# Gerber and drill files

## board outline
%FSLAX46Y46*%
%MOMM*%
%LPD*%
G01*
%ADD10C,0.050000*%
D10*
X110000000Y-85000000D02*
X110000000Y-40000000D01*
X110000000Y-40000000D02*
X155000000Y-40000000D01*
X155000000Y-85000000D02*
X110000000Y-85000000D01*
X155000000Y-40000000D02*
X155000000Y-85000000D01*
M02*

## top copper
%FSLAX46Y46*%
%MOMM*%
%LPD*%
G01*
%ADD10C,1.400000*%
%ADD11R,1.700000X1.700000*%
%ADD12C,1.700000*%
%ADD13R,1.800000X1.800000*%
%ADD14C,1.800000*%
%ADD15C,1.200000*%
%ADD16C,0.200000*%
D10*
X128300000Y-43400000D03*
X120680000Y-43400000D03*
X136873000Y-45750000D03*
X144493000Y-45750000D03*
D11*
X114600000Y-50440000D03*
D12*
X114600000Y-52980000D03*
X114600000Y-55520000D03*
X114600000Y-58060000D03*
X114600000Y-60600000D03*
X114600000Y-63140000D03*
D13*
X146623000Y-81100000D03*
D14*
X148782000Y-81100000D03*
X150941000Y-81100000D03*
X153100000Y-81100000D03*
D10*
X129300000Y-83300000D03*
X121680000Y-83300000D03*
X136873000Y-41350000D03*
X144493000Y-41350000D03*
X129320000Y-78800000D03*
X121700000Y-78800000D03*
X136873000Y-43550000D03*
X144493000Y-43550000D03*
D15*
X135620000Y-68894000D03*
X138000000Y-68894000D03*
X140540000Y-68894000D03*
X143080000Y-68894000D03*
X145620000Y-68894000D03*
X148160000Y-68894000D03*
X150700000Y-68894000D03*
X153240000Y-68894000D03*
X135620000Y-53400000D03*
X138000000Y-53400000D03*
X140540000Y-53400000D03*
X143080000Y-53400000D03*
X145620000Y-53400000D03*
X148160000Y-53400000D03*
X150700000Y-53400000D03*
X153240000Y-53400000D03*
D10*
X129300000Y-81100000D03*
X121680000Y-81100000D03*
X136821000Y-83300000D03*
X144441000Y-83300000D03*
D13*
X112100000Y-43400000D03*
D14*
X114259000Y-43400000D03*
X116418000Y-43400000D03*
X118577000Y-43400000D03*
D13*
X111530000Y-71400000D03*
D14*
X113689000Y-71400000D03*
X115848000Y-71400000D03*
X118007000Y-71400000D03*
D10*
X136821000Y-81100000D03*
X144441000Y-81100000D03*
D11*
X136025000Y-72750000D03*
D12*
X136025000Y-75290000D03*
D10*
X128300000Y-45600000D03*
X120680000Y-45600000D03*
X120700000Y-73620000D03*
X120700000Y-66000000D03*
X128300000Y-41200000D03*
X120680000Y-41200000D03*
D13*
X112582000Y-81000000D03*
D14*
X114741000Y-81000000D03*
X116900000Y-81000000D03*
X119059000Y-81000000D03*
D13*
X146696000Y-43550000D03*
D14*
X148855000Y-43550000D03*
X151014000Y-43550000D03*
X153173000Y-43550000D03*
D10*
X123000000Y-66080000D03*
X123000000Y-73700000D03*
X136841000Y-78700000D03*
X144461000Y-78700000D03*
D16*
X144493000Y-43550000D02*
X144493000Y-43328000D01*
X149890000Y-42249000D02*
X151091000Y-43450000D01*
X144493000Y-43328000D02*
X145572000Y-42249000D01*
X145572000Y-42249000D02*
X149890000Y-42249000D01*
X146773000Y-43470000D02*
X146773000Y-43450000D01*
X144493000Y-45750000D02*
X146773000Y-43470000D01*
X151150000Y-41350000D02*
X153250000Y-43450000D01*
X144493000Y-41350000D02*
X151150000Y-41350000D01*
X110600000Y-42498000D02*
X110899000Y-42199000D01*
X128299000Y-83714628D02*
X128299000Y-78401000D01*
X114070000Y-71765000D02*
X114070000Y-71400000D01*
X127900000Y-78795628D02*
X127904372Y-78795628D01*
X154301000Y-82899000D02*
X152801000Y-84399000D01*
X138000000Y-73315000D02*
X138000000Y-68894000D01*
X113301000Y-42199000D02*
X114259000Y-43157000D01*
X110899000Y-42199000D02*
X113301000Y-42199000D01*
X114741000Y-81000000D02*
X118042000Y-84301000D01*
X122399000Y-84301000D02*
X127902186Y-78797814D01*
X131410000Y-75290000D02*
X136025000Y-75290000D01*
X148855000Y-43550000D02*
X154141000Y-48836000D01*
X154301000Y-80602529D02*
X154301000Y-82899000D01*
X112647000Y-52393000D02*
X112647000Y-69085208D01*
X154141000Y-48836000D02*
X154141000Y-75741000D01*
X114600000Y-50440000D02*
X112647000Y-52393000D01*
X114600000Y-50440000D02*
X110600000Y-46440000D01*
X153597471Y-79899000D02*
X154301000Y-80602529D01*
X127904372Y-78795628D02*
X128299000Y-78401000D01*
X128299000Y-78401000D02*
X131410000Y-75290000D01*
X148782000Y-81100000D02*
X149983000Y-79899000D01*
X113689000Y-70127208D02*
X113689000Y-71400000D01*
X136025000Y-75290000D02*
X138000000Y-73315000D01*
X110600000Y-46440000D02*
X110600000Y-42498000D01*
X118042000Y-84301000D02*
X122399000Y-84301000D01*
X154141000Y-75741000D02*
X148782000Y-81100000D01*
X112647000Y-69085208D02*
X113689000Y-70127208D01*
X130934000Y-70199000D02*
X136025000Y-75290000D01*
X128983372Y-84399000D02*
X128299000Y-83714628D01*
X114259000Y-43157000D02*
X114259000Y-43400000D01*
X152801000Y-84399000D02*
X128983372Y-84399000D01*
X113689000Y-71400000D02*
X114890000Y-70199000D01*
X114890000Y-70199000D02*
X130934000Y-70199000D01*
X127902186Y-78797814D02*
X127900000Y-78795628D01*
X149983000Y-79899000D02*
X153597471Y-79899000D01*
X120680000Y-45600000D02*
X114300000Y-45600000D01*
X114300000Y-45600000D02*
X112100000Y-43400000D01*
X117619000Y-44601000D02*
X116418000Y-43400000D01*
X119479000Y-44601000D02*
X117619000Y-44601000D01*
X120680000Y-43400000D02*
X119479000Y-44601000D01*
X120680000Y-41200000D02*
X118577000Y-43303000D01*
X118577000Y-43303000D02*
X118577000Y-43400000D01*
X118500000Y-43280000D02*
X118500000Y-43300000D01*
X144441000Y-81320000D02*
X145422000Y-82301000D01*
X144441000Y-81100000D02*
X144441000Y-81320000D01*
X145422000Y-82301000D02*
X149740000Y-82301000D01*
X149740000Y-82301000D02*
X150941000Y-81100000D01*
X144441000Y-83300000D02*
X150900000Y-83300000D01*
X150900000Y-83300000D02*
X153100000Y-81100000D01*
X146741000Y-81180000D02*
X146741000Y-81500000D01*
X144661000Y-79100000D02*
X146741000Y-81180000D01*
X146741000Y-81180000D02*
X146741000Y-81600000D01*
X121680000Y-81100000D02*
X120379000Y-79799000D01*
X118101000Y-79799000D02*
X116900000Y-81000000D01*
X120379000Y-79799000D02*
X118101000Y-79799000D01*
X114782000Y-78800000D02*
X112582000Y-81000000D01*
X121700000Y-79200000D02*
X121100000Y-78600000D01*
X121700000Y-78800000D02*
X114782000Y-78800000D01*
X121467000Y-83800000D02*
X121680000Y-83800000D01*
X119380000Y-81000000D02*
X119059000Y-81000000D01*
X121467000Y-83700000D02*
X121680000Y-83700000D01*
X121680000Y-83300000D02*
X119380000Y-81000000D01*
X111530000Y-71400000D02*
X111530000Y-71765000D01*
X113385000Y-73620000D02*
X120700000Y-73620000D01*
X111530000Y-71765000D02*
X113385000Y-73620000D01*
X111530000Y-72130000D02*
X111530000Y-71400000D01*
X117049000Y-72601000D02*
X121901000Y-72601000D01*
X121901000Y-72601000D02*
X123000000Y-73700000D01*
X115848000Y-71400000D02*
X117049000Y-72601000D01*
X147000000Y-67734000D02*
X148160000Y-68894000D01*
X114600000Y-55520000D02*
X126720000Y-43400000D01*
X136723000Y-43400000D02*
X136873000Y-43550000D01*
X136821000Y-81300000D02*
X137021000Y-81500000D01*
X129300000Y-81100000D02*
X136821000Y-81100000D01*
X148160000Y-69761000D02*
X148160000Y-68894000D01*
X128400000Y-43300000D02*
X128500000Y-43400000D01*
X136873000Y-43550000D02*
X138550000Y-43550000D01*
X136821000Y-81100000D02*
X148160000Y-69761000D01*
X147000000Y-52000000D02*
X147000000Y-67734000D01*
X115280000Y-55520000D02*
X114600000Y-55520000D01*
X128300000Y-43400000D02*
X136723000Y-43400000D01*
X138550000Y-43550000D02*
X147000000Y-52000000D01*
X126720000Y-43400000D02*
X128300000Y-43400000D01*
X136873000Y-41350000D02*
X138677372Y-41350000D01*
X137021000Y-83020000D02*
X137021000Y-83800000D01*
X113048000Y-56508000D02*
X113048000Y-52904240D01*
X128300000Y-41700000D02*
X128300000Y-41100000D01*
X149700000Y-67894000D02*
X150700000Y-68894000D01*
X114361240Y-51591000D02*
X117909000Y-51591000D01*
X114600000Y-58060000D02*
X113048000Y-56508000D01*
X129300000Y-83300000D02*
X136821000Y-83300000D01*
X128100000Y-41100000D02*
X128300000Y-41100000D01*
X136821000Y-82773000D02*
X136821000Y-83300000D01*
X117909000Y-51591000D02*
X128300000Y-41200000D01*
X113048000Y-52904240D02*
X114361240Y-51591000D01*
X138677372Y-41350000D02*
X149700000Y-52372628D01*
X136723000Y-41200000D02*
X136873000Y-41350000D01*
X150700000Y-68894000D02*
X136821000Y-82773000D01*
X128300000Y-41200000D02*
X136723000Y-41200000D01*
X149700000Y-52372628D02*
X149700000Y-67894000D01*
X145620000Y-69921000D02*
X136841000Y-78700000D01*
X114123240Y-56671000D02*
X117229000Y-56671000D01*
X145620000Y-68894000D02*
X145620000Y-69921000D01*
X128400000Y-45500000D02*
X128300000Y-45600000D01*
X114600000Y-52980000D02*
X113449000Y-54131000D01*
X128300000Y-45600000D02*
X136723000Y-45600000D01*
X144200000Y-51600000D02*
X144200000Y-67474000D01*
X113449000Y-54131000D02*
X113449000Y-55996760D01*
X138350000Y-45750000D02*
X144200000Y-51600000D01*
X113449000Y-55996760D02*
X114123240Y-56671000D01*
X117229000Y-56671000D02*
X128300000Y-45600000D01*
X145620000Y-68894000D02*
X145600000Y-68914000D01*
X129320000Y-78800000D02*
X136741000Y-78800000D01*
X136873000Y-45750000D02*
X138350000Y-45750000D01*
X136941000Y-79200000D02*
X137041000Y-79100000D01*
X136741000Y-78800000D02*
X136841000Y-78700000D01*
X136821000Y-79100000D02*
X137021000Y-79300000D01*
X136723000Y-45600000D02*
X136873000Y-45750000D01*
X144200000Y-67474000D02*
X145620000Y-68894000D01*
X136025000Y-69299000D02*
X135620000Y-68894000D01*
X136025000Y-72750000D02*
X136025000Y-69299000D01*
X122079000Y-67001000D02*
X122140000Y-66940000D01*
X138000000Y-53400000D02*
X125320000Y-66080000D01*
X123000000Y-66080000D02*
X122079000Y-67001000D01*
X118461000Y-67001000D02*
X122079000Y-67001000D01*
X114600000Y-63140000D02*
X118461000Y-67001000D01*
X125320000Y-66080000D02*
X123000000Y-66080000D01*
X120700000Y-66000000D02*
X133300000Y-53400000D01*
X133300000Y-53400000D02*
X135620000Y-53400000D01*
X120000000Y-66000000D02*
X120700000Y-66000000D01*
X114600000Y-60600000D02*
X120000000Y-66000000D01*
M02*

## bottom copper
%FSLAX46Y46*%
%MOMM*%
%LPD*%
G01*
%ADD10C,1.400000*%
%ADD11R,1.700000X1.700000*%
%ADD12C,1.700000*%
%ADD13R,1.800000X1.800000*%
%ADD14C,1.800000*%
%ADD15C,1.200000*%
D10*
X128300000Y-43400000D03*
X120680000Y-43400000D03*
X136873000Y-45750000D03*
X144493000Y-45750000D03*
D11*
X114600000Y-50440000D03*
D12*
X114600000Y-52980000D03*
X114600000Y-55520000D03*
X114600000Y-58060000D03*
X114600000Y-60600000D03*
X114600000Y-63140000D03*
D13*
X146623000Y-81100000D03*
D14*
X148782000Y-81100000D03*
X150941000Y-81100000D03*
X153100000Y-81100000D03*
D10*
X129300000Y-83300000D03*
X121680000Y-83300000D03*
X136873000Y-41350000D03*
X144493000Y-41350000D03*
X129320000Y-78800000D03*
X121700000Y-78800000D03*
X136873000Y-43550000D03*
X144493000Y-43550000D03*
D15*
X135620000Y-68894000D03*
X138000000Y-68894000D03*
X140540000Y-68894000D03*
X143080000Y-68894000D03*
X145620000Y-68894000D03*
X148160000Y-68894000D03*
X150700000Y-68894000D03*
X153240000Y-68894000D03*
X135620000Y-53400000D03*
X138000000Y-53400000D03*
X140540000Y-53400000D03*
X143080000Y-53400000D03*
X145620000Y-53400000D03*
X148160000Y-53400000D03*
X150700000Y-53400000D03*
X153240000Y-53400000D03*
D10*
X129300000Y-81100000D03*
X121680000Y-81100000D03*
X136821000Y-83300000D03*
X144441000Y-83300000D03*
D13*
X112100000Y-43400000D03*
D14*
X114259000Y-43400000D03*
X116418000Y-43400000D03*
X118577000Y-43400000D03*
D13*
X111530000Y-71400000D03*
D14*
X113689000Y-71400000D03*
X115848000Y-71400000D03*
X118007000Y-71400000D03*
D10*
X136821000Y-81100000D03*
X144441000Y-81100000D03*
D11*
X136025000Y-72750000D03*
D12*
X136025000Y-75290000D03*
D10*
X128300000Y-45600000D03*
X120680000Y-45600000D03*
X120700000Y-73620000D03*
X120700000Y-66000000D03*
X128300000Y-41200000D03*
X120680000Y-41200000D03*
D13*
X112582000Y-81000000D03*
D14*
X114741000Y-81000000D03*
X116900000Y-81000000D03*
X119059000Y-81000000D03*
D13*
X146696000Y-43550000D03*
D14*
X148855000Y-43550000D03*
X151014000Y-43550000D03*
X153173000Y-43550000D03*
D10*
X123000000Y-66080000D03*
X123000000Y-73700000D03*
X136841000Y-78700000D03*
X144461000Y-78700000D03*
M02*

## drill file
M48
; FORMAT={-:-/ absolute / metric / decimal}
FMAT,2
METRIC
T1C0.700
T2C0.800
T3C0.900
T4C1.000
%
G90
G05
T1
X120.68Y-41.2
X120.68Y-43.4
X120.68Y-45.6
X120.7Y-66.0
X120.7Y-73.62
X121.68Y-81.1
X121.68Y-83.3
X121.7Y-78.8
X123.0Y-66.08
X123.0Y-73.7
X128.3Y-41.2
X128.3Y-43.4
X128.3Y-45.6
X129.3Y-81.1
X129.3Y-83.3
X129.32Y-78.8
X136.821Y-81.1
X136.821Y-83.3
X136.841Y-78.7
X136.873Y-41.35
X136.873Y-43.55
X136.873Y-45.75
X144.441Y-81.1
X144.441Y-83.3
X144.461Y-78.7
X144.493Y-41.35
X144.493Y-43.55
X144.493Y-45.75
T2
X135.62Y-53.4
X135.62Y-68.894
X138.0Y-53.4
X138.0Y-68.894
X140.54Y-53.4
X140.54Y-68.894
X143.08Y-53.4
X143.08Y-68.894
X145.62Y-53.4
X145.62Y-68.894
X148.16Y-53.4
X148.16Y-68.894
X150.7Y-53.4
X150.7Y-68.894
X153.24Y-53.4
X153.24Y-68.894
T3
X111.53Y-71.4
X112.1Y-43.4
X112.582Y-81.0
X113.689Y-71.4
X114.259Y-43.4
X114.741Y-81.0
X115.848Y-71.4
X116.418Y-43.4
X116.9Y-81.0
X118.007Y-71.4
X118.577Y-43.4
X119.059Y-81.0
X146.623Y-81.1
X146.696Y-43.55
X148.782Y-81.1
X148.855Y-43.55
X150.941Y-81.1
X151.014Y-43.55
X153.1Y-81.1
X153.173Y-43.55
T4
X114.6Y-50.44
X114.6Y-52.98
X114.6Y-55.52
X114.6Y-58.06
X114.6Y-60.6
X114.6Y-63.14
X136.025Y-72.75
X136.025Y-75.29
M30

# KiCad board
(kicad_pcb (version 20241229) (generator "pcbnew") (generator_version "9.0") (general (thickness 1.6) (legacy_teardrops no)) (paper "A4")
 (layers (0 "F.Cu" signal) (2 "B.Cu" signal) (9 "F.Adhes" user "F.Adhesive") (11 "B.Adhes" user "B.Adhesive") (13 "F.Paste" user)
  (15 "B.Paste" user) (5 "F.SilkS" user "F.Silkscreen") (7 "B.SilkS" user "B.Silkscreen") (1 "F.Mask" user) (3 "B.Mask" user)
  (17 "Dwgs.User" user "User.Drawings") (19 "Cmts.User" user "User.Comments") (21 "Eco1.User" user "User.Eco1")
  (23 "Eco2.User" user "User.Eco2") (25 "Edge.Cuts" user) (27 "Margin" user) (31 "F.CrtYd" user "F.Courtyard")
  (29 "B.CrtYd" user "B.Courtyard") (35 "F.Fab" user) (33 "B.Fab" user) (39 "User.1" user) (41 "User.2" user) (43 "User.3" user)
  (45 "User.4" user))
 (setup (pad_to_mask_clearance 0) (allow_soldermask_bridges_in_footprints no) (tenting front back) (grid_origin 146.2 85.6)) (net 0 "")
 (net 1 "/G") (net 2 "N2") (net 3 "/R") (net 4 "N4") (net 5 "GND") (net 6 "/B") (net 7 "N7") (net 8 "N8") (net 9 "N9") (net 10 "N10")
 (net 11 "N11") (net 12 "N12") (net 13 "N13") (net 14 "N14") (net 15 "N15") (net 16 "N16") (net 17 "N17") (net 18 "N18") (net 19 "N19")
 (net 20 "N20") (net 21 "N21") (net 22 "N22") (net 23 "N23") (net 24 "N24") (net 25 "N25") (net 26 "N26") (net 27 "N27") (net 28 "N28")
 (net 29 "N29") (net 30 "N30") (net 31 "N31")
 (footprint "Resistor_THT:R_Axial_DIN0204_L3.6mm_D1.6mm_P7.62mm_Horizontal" (layer "F.Cu") (at 128.3 43.4 180)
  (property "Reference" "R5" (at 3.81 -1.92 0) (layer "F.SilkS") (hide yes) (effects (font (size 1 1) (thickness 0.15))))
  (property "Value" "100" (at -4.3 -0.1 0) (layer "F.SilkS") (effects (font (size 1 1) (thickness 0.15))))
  (pad "1" thru_hole circle (at 0 0 180) (size 1.4 1.4) (drill 0.7) (layers "*.Cu" "*.Mask") (remove_unused_layers no) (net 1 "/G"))
  (pad "2" thru_hole circle (at 7.62 0 180) (size 1.4 1.4) (drill 0.7) (layers "*.Cu" "*.Mask") (remove_unused_layers no) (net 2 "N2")))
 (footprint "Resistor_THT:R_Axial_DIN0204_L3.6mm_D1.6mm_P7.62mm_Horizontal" (layer "F.Cu") (at 136.873 45.75)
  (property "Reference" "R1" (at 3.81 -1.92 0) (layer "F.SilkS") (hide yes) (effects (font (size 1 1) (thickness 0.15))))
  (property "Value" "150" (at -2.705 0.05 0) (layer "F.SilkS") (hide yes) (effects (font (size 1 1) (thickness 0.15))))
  (pad "1" thru_hole circle (at 0 0) (size 1.4 1.4) (drill 0.7) (layers "*.Cu" "*.Mask") (remove_unused_layers no) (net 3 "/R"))
  (pad "2" thru_hole circle (at 7.62 0) (size 1.4 1.4) (drill 0.7) (layers "*.Cu" "*.Mask") (remove_unused_layers no) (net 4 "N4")))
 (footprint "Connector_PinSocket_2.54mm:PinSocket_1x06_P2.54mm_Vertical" (layer "F.Cu") (at 114.6 50.44)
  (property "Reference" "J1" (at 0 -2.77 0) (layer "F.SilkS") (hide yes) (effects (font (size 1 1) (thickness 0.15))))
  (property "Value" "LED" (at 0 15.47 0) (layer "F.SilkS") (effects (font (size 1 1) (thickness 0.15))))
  (pad "1" thru_hole rect (at 0 0) (size 1.7 1.7) (drill 1) (layers "*.Cu" "*.Mask") (remove_unused_layers no) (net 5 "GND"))
  (pad "2" thru_hole circle (at 0 2.54) (size 1.7 1.7) (drill 1) (layers "*.Cu" "*.Mask") (remove_unused_layers no) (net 3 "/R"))
  (pad "3" thru_hole circle (at 0 5.08) (size 1.7 1.7) (drill 1) (layers "*.Cu" "*.Mask") (remove_unused_layers no) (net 1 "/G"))
  (pad "4" thru_hole circle (at 0 7.62) (size 1.7 1.7) (drill 1) (layers "*.Cu" "*.Mask") (remove_unused_layers no) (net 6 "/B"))
  (pad "5" thru_hole circle (at 0 10.16) (size 1.7 1.7) (drill 1) (layers "*.Cu" "*.Mask") (remove_unused_layers no) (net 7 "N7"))
  (pad "6" thru_hole circle (at 0 12.7) (size 1.7 1.7) (drill 1) (layers "*.Cu" "*.Mask") (remove_unused_layers no) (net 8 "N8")))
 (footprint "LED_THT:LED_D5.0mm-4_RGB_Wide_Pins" (layer "F.Cu") (at 146.623 81.1)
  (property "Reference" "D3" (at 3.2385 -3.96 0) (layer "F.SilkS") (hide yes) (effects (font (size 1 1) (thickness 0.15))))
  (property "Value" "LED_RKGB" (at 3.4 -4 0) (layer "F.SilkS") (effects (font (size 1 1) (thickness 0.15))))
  (pad "1" thru_hole rect (at 0 0) (size 1.8 1.8) (drill 0.9) (layers "*.Cu" "*.Mask") (remove_unused_layers no) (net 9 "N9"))
  (pad "2" thru_hole circle (at 2.159 0) (size 1.8 1.8) (drill 0.9) (layers "*.Cu" "*.Mask") (remove_unused_layers no) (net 5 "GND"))
  (pad "3" thru_hole circle (at 4.318 0) (size 1.8 1.8) (drill 0.9) (layers "*.Cu" "*.Mask") (remove_unused_layers no) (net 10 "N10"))
  (pad "4" thru_hole circle (at 6.477 0) (size 1.8 1.8) (drill 0.9) (layers "*.Cu" "*.Mask") (remove_unused_layers no) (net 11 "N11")))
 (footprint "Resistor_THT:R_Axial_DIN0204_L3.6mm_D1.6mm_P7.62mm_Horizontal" (layer "F.Cu") (at 129.3 83.3 180)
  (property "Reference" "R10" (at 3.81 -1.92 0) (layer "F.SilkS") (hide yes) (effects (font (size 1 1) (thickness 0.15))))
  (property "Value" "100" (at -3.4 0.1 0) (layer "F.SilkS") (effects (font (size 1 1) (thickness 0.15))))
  (pad "1" thru_hole circle (at 0 0 180) (size 1.4 1.4) (drill 0.7) (layers "*.Cu" "*.Mask") (remove_unused_layers no) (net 6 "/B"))
  (pad "2" thru_hole circle (at 7.62 0 180) (size 1.4 1.4) (drill 0.7) (layers "*.Cu" "*.Mask") (remove_unused_layers no) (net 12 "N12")))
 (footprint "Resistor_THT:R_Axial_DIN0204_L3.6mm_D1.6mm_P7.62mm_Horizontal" (layer "F.Cu") (at 136.873 41.35)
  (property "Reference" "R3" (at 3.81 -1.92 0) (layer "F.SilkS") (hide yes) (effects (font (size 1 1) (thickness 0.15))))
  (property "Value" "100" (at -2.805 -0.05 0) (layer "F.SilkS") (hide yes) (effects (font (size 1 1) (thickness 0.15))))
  (pad "1" thru_hole circle (at 0 0) (size 1.4 1.4) (drill 0.7) (layers "*.Cu" "*.Mask") (remove_unused_layers no) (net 6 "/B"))
  (pad "2" thru_hole circle (at 7.62 0) (size 1.4 1.4) (drill 0.7) (layers "*.Cu" "*.Mask") (remove_unused_layers no) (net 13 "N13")))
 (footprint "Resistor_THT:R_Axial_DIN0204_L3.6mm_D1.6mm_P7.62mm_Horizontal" (layer "F.Cu") (at 129.32 78.8 180)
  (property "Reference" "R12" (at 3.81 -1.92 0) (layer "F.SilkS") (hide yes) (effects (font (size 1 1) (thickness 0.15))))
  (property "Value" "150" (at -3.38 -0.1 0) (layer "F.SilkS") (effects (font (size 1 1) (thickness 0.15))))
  (pad "1" thru_hole circle (at 0 0 180) (size 1.4 1.4) (drill 0.7) (layers "*.Cu" "*.Mask") (remove_unused_layers no) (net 3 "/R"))
  (pad "2" thru_hole circle (at 7.62 0 180) (size 1.4 1.4) (drill 0.7) (layers "*.Cu" "*.Mask") (remove_unused_layers no) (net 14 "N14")))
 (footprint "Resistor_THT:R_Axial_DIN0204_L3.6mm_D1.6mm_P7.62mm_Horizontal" (layer "F.Cu") (at 136.873 43.55)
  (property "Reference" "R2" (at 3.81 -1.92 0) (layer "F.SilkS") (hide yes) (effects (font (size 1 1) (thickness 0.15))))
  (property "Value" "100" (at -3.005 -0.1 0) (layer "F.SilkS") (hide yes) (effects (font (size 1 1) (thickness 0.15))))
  (pad "1" thru_hole circle (at 0 0) (size 1.4 1.4) (drill 0.7) (layers "*.Cu" "*.Mask") (remove_unused_layers no) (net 1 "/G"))
  (pad "2" thru_hole circle (at 7.62 0) (size 1.4 1.4) (drill 0.7) (layers "*.Cu" "*.Mask") (remove_unused_layers no) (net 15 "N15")))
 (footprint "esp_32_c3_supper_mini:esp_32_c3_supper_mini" (layer "F.Cu") (at 145.62 61.274 90)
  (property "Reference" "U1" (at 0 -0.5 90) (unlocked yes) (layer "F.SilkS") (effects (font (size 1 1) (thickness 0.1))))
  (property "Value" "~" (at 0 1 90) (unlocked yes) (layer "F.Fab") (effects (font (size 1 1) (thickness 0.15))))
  (pad "1" thru_hole circle (at -7.62 -10 90) (size 1.2 1.2) (drill 0.8) (layers "*.Cu" "*.Mask") (remove_unused_layers no) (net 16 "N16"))
  (pad "2" thru_hole circle (at -7.62 -7.62 90) (size 1.2 1.2) (drill 0.8) (layers "*.Cu" "*.Mask") (remove_unused_layers no) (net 5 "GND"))
  (pad "3" thru_hole circle (at -7.62 -5.08 90) (size 1.2 1.2) (drill 0.8) (layers "*.Cu" "*.Mask") (remove_unused_layers no) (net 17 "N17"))
  (pad "4" thru_hole circle (at -7.62 -2.54 90) (size 1.2 1.2) (drill 0.8) (layers "*.Cu" "*.Mask") (remove_unused_layers no) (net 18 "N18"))
  (pad "5" thru_hole circle (at -7.62 0 90) (size 1.2 1.2) (drill 0.8) (layers "*.Cu" "*.Mask") (remove_unused_layers no) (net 3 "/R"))
  (pad "6" thru_hole circle (at -7.62 2.54 90) (size 1.2 1.2) (drill 0.8) (layers "*.Cu" "*.Mask") (remove_unused_layers no) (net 1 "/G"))
  (pad "7" thru_hole circle (at -7.62 5.08 90) (size 1.2 1.2) (drill 0.8) (layers "*.Cu" "*.Mask") (remove_unused_layers no) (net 6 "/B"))
  (pad "8" thru_hole circle (at -7.62 7.62 90) (size 1.2 1.2) (drill 0.8) (layers "*.Cu" "*.Mask") (remove_unused_layers no) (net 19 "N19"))
  (pad "9" thru_hole circle (at 7.874 -10 90) (size 1.2 1.2) (drill 0.8) (layers "*.Cu" "*.Mask") (remove_unused_layers no) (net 7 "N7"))
  (pad "10" thru_hole circle (at 7.874 -7.62 90) (size 1.2 1.2) (drill 0.8) (layers "*.Cu" "*.Mask") (remove_unused_layers no) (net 8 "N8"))
  (pad "11" thru_hole circle (at 7.874 -5.08 90) (size 1.2 1.2) (drill 0.8) (layers "*.Cu" "*.Mask") (remove_unused_layers no)
   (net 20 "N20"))
  (pad "12" thru_hole circle (at 7.874 -2.54 90) (size 1.2 1.2) (drill 0.8) (layers "*.Cu" "*.Mask") (remove_unused_layers no)
   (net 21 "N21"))
  (pad "13" thru_hole circle (at 7.874 0 90) (size 1.2 1.2) (drill 0.8) (layers "*.Cu" "*.Mask") (remove_unused_layers no) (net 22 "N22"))
  (pad "14" thru_hole circle (at 7.874 2.54 90) (size 1.2 1.2) (drill 0.8) (layers "*.Cu" "*.Mask") (remove_unused_layers no) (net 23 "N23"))
  (pad "15" thru_hole circle (at 7.874 5.08 90) (size 1.2 1.2) (drill 0.8) (layers "*.Cu" "*.Mask") (remove_unused_layers no) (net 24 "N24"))
  (pad "16" thru_hole circle (at 7.874 7.62 90) (size 1.2 1.2) (drill 0.8) (layers "*.Cu" "*.Mask") (remove_unused_layers no) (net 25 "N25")))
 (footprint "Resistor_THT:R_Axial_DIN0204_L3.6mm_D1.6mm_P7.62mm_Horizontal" (layer "F.Cu") (at 129.3 81.1 180)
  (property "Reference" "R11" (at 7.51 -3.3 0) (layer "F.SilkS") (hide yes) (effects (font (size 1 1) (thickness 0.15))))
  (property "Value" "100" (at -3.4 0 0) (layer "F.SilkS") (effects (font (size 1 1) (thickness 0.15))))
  (pad "1" thru_hole circle (at 0 0 180) (size 1.4 1.4) (drill 0.7) (layers "*.Cu" "*.Mask") (remove_unused_layers no) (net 1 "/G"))
  (pad "2" thru_hole circle (at 7.62 0 180) (size 1.4 1.4) (drill 0.7) (layers "*.Cu" "*.Mask") (remove_unused_layers no) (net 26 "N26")))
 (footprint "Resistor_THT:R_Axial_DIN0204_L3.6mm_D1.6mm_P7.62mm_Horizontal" (layer "F.Cu") (at 136.821 83.3)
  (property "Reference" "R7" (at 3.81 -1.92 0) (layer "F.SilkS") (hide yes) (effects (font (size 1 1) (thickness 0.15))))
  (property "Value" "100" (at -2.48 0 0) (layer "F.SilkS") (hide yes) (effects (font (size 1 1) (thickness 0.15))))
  (pad "1" thru_hole circle (at 0 0) (size 1.4 1.4) (drill 0.7) (layers "*.Cu" "*.Mask") (remove_unused_layers no) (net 6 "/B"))
  (pad "2" thru_hole circle (at 7.62 0) (size 1.4 1.4) (drill 0.7) (layers "*.Cu" "*.Mask") (remove_unused_layers no) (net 11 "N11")))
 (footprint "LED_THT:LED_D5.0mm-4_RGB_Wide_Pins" (layer "F.Cu") (at 112.1 43.4)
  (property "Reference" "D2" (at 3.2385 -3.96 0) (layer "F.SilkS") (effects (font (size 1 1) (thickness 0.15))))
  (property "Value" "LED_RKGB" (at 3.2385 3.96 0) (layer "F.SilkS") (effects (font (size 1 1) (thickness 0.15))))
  (pad "1" thru_hole rect (at 0 0) (size 1.8 1.8) (drill 0.9) (layers "*.Cu" "*.Mask") (remove_unused_layers no) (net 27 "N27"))
  (pad "2" thru_hole circle (at 2.159 0) (size 1.8 1.8) (drill 0.9) (layers "*.Cu" "*.Mask") (remove_unused_layers no) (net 5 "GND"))
  (pad "3" thru_hole circle (at 4.318 0) (size 1.8 1.8) (drill 0.9) (layers "*.Cu" "*.Mask") (remove_unused_layers no) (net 2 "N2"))
  (pad "4" thru_hole circle (at 6.477 0) (size 1.8 1.8) (drill 0.9) (layers "*.Cu" "*.Mask") (remove_unused_layers no) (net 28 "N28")))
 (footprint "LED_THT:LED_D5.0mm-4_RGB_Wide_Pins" (layer "F.Cu") (at 111.53 71.4)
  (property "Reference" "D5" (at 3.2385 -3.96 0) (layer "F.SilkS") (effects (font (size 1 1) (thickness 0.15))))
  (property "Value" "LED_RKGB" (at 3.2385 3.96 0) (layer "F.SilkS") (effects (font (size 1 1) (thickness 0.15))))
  (pad "1" thru_hole rect (at 0 0) (size 1.8 1.8) (drill 0.9) (layers "*.Cu" "*.Mask") (remove_unused_layers no) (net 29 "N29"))
  (pad "2" thru_hole circle (at 2.159 0) (size 1.8 1.8) (drill 0.9) (layers "*.Cu" "*.Mask") (remove_unused_layers no) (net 5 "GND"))
  (pad "3" thru_hole circle (at 4.318 0) (size 1.8 1.8) (drill 0.9) (layers "*.Cu" "*.Mask") (remove_unused_layers no) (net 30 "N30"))
  (pad "4" thru_hole circle (at 6.477 0) (size 1.8 1.8) (drill 0.9) (layers "*.Cu" "*.Mask") (remove_unused_layers no) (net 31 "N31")))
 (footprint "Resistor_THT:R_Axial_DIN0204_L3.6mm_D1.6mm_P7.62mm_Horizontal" (layer "F.Cu") (at 136.821 81.1)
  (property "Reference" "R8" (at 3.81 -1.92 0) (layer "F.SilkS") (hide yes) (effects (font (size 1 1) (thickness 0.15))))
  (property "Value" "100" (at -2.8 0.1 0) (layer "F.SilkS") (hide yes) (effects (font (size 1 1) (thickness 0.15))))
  (pad "1" thru_hole circle (at 0 0) (size 1.4 1.4) (drill 0.7) (layers "*.Cu" "*.Mask") (remove_unused_layers no) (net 1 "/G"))
  (pad "2" thru_hole circle (at 7.62 0) (size 1.4 1.4) (drill 0.7) (layers "*.Cu" "*.Mask") (remove_unused_layers no) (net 10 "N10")))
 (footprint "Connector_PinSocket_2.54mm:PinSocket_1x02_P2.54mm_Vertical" (layer "F.Cu") (at 136.025 72.75)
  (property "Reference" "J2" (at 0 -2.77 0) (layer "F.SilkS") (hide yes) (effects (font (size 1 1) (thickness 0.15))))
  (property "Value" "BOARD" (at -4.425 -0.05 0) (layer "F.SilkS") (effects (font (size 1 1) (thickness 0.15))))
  (pad "1" thru_hole rect (at 0 0) (size 1.7 1.7) (drill 1) (layers "*.Cu" "*.Mask") (remove_unused_layers no) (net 16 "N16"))
  (pad "2" thru_hole circle (at 0 2.54) (size 1.7 1.7) (drill 1) (layers "*.Cu" "*.Mask") (remove_unused_layers no) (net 5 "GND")))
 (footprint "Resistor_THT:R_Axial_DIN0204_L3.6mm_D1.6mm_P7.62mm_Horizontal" (layer "F.Cu") (at 128.3 45.6 180)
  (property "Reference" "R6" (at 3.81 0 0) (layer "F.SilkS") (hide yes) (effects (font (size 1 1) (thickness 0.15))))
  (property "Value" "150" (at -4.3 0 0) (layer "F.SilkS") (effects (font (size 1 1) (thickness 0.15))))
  (pad "1" thru_hole circle (at 0 0 180) (size 1.4 1.4) (drill 0.7) (layers "*.Cu" "*.Mask") (remove_unused_layers no) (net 3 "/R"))
  (pad "2" thru_hole circle (at 7.62 0 180) (size 1.4 1.4) (drill 0.7) (layers "*.Cu" "*.Mask") (remove_unused_layers no) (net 27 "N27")))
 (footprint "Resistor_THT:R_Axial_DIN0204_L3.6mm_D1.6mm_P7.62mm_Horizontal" (layer "F.Cu") (at 120.7 73.62 90)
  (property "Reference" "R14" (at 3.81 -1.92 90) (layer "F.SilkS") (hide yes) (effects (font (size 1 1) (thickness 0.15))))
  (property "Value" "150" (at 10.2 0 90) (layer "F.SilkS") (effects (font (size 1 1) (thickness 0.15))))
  (pad "1" thru_hole circle (at 0 0 90) (size 1.4 1.4) (drill 0.7) (layers "*.Cu" "*.Mask") (remove_unused_layers no) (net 29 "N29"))
  (pad "2" thru_hole circle (at 7.62 0 90) (size 1.4 1.4) (drill 0.7) (layers "*.Cu" "*.Mask") (remove_unused_layers no) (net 7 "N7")))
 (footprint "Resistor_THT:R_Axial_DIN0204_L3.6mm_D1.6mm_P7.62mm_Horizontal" (layer "F.Cu") (at 128.3 41.2 180)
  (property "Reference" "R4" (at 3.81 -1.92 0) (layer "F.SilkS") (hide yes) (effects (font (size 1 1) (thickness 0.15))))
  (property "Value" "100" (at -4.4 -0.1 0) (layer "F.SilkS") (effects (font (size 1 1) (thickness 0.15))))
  (pad "1" thru_hole circle (at 0 0 180) (size 1.4 1.4) (drill 0.7) (layers "*.Cu" "*.Mask") (remove_unused_layers no) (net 6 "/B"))
  (pad "2" thru_hole circle (at 7.62 0 180) (size 1.4 1.4) (drill 0.7) (layers "*.Cu" "*.Mask") (remove_unused_layers no) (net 28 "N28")))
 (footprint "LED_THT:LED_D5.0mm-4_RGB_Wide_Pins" (layer "F.Cu") (at 112.582 81)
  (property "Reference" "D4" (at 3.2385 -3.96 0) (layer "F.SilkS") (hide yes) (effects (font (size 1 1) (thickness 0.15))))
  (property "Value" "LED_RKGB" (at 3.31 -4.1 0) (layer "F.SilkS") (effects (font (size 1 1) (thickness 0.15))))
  (pad "1" thru_hole rect (at 0 0) (size 1.8 1.8) (drill 0.9) (layers "*.Cu" "*.Mask") (remove_unused_layers no) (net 14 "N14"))
  (pad "2" thru_hole circle (at 2.159 0) (size 1.8 1.8) (drill 0.9) (layers "*.Cu" "*.Mask") (remove_unused_layers no) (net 5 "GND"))
  (pad "3" thru_hole circle (at 4.318 0) (size 1.8 1.8) (drill 0.9) (layers "*.Cu" "*.Mask") (remove_unused_layers no) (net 26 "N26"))
  (pad "4" thru_hole circle (at 6.477 0) (size 1.8 1.8) (drill 0.9) (layers "*.Cu" "*.Mask") (remove_unused_layers no) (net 12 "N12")))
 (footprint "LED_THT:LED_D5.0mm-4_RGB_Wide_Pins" (layer "F.Cu") (at 146.696 43.55)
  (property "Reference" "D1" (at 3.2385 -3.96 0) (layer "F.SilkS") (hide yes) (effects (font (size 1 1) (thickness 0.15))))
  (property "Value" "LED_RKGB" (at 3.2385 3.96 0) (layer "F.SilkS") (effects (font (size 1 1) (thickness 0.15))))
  (pad "1" thru_hole rect (at 0 0) (size 1.8 1.8) (drill 0.9) (layers "*.Cu" "*.Mask") (remove_unused_layers no) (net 4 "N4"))
  (pad "2" thru_hole circle (at 2.159 0) (size 1.8 1.8) (drill 0.9) (layers "*.Cu" "*.Mask") (remove_unused_layers no) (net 5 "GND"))
  (pad "3" thru_hole circle (at 4.318 0) (size 1.8 1.8) (drill 0.9) (layers "*.Cu" "*.Mask") (remove_unused_layers no) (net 15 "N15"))
  (pad "4" thru_hole circle (at 6.477 0) (size 1.8 1.8) (drill 0.9) (layers "*.Cu" "*.Mask") (remove_unused_layers no) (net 13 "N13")))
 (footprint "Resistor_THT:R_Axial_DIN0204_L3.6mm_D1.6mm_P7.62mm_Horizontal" (layer "F.Cu") (at 123 66.08 -90)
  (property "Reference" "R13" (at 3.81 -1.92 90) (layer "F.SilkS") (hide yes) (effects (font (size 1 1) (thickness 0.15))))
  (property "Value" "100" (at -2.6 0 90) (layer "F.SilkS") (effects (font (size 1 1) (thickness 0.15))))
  (pad "1" thru_hole circle (at 0 0 270) (size 1.4 1.4) (drill 0.7) (layers "*.Cu" "*.Mask") (remove_unused_layers no) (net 8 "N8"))
  (pad "2" thru_hole circle (at 7.62 0 270) (size 1.4 1.4) (drill 0.7) (layers "*.Cu" "*.Mask") (remove_unused_layers no) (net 30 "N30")))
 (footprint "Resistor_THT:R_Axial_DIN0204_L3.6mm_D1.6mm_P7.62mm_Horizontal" (layer "F.Cu") (at 136.841 78.7)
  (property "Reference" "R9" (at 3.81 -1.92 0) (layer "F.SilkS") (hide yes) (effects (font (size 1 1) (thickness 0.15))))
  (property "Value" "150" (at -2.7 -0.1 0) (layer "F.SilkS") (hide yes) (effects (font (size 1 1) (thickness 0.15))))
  (pad "1" thru_hole circle (at 0 0) (size 1.4 1.4) (drill 0.7) (layers "*.Cu" "*.Mask") (remove_unused_layers no) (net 3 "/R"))
  (pad "2" thru_hole circle (at 7.62 0) (size 1.4 1.4) (drill 0.7) (layers "*.Cu" "*.Mask") (remove_unused_layers no) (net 9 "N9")))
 (gr_line (start 110 85) (end 110 40) (stroke (width 0.05) (type default)) (layer "Edge.Cuts"))
 (gr_line (start 110 40) (end 155 40) (stroke (width 0.05) (type default)) (layer "Edge.Cuts"))
 (gr_line (start 155 85) (end 110 85) (stroke (width 0.05) (type default)) (layer "Edge.Cuts"))
 (gr_line (start 155 40) (end 155 85) (stroke (width 0.05) (type default)) (layer "Edge.Cuts"))
 (segment (start 144.493 43.55) (end 144.493 43.328) (width 0.2) (layer "F.Cu") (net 15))
 (segment (start 149.89 42.249) (end 151.091 43.45) (width 0.2) (layer "F.Cu") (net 15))
 (segment (start 144.493 43.328) (end 145.572 42.249) (width 0.2) (layer "F.Cu") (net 15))
 (segment (start 145.572 42.249) (end 149.89 42.249) (width 0.2) (layer "F.Cu") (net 15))
 (segment (start 146.773 43.47) (end 146.773 43.45) (width 0.2) (layer "F.Cu") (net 4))
 (segment (start 144.493 45.75) (end 146.773 43.47) (width 0.2) (layer "F.Cu") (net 4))
 (segment (start 151.15 41.35) (end 153.25 43.45) (width 0.2) (layer "F.Cu") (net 13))
 (segment (start 144.493 41.35) (end 151.15 41.35) (width 0.2) (layer "F.Cu") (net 13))
 (segment (start 110.6 42.498) (end 110.899 42.199) (width 0.2) (layer "F.Cu") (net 5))
 (segment (start 128.299 83.714628) (end 128.299 78.401) (width 0.2) (layer "F.Cu") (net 5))
 (segment (start 114.07 71.765) (end 114.07 71.4) (width 0.2) (layer "F.Cu") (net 5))
 (segment (start 127.9 78.795628) (end 127.904372 78.795628) (width 0.2) (layer "F.Cu") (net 5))
 (segment (start 154.301 82.899) (end 152.801 84.399) (width 0.2) (layer "F.Cu") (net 5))
 (segment (start 138 73.315) (end 138 68.894) (width 0.2) (layer "F.Cu") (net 5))
 (segment (start 113.301 42.199) (end 114.259 43.157) (width 0.2) (layer "F.Cu") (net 5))
 (segment (start 110.899 42.199) (end 113.301 42.199) (width 0.2) (layer "F.Cu") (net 5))
 (segment (start 114.741 81) (end 118.042 84.301) (width 0.2) (layer "F.Cu") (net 5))
 (segment (start 122.399 84.301) (end 127.902186 78.797814) (width 0.2) (layer "F.Cu") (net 5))
 (segment (start 131.41 75.29) (end 136.025 75.29) (width 0.2) (layer "F.Cu") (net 5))
 (segment (start 148.855 43.55) (end 154.141 48.836) (width 0.2) (layer "F.Cu") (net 5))
 (segment (start 154.301 80.602529) (end 154.301 82.899) (width 0.2) (layer "F.Cu") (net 5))
 (segment (start 112.647 52.393) (end 112.647 69.085208) (width 0.2) (layer "F.Cu") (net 5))
 (segment (start 154.141 48.836) (end 154.141 75.741) (width 0.2) (layer "F.Cu") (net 5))
 (segment (start 114.6 50.44) (end 112.647 52.393) (width 0.2) (layer "F.Cu") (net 5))
 (segment (start 114.6 50.44) (end 110.6 46.44) (width 0.2) (layer "F.Cu") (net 5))
 (segment (start 153.597471 79.899) (end 154.301 80.602529) (width 0.2) (layer "F.Cu") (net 5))
 (segment (start 127.904372 78.795628) (end 128.299 78.401) (width 0.2) (layer "F.Cu") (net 5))
 (segment (start 128.299 78.401) (end 131.41 75.29) (width 0.2) (layer "F.Cu") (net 5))
 (segment (start 148.782 81.1) (end 149.983 79.899) (width 0.2) (layer "F.Cu") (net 5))
 (segment (start 113.689 70.127208) (end 113.689 71.4) (width 0.2) (layer "F.Cu") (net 5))
 (segment (start 136.025 75.29) (end 138 73.315) (width 0.2) (layer "F.Cu") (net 5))
 (segment (start 110.6 46.44) (end 110.6 42.498) (width 0.2) (layer "F.Cu") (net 5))
 (segment (start 118.042 84.301) (end 122.399 84.301) (width 0.2) (layer "F.Cu") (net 5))
 (segment (start 154.141 75.741) (end 148.782 81.1) (width 0.2) (layer "F.Cu") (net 5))
 (segment (start 112.647 69.085208) (end 113.689 70.127208) (width 0.2) (layer "F.Cu") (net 5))
 (segment (start 130.934 70.199) (end 136.025 75.29) (width 0.2) (layer "F.Cu") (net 5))
 (segment (start 128.983372 84.399) (end 128.299 83.714628) (width 0.2) (layer "F.Cu") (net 5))
 (segment (start 114.259 43.157) (end 114.259 43.4) (width 0.2) (layer "F.Cu") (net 5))
 (segment (start 152.801 84.399) (end 128.983372 84.399) (width 0.2) (layer "F.Cu") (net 5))
 (segment (start 113.689 71.4) (end 114.89 70.199) (width 0.2) (layer "F.Cu") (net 5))
 (segment (start 114.89 70.199) (end 130.934 70.199) (width 0.2) (layer "F.Cu") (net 5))
 (segment (start 127.902186 78.797814) (end 127.9 78.795628) (width 0.2) (layer "F.Cu") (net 5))
 (segment (start 149.983 79.899) (end 153.597471 79.899) (width 0.2) (layer "F.Cu") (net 5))
 (segment (start 120.68 45.6) (end 114.3 45.6) (width 0.2) (layer "F.Cu") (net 27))
 (segment (start 114.3 45.6) (end 112.1 43.4) (width 0.2) (layer "F.Cu") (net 27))
 (segment (start 117.619 44.601) (end 116.418 43.4) (width 0.2) (layer "F.Cu") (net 2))
 (segment (start 119.479 44.601) (end 117.619 44.601) (width 0.2) (layer "F.Cu") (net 2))
 (segment (start 120.68 43.4) (end 119.479 44.601) (width 0.2) (layer "F.Cu") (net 2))
 (segment (start 120.68 41.2) (end 118.577 43.303) (width 0.2) (layer "F.Cu") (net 28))
 (segment (start 118.577 43.303) (end 118.577 43.4) (width 0.2) (layer "F.Cu") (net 28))
 (segment (start 118.5 43.28) (end 118.5 43.3) (width 0.2) (layer "F.Cu") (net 28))
 (segment (start 144.441 81.32) (end 145.422 82.301) (width 0.2) (layer "F.Cu") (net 10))
 (segment (start 144.441 81.1) (end 144.441 81.32) (width 0.2) (layer "F.Cu") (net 10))
 (segment (start 145.422 82.301) (end 149.74 82.301) (width 0.2) (layer "F.Cu") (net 10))
 (segment (start 149.74 82.301) (end 150.941 81.1) (width 0.2) (layer "F.Cu") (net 10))
 (segment (start 144.441 83.3) (end 150.9 83.3) (width 0.2) (layer "F.Cu") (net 11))
 (segment (start 150.9 83.3) (end 153.1 81.1) (width 0.2) (layer "F.Cu") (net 11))
 (segment (start 146.741 81.18) (end 146.741 81.5) (width 0.2) (layer "F.Cu") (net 9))
 (segment (start 144.661 79.1) (end 146.741 81.18) (width 0.2) (layer "F.Cu") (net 9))
 (segment (start 146.741 81.18) (end 146.741 81.6) (width 0.2) (layer "F.Cu") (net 9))
 (segment (start 121.68 81.1) (end 120.379 79.799) (width 0.2) (layer "F.Cu") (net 26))
 (segment (start 118.101 79.799) (end 116.9 81) (width 0.2) (layer "F.Cu") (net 26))
 (segment (start 120.379 79.799) (end 118.101 79.799) (width 0.2) (layer "F.Cu") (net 26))
 (segment (start 114.782 78.8) (end 112.582 81) (width 0.2) (layer "F.Cu") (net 14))
 (segment (start 121.7 79.2) (end 121.1 78.6) (width 0.2) (layer "F.Cu") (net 14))
 (segment (start 121.7 78.8) (end 114.782 78.8) (width 0.2) (layer "F.Cu") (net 14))
 (segment (start 121.467 83.8) (end 121.68 83.8) (width 0.2) (layer "F.Cu") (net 12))
 (segment (start 119.38 81) (end 119.059 81) (width 0.2) (layer "F.Cu") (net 12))
 (segment (start 121.467 83.7) (end 121.68 83.7) (width 0.2) (layer "F.Cu") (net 12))
 (segment (start 121.68 83.3) (end 119.38 81) (width 0.2) (layer "F.Cu") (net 12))
 (segment (start 111.53 71.4) (end 111.53 71.765) (width 0.2) (layer "F.Cu") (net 29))
 (segment (start 113.385 73.62) (end 120.7 73.62) (width 0.2) (layer "F.Cu") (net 29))
 (segment (start 111.53 71.765) (end 113.385 73.62) (width 0.2) (layer "F.Cu") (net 29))
 (segment (start 111.53 72.13) (end 111.53 71.4) (width 0.2) (layer "F.Cu") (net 29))
 (segment (start 117.049 72.601) (end 121.901 72.601) (width 0.2) (layer "F.Cu") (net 30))
 (segment (start 121.901 72.601) (end 123 73.7) (width 0.2) (layer "F.Cu") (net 30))
 (segment (start 115.848 71.4) (end 117.049 72.601) (width 0.2) (layer "F.Cu") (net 30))
 (segment (start 147 67.734) (end 148.16 68.894) (width 0.2) (layer "F.Cu") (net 1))
 (segment (start 114.6 55.52) (end 126.72 43.4) (width 0.2) (layer "F.Cu") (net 1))
 (segment (start 136.723 43.4) (end 136.873 43.55) (width 0.2) (layer "F.Cu") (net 1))
 (segment (start 136.821 81.3) (end 137.021 81.5) (width 0.2) (layer "F.Cu") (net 1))
 (segment (start 129.3 81.1) (end 136.821 81.1) (width 0.2) (layer "F.Cu") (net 1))
 (segment (start 148.16 69.761) (end 148.16 68.894) (width 0.2) (layer "F.Cu") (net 1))
 (segment (start 128.4 43.3) (end 128.5 43.4) (width 0.2) (layer "F.Cu") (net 1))
 (segment (start 136.873 43.55) (end 138.55 43.55) (width 0.2) (layer "F.Cu") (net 1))
 (segment (start 136.821 81.1) (end 148.16 69.761) (width 0.2) (layer "F.Cu") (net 1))
 (segment (start 147 52) (end 147 67.734) (width 0.2) (layer "F.Cu") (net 1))
 (segment (start 115.28 55.52) (end 114.6 55.52) (width 0.2) (layer "F.Cu") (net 1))
 (segment (start 128.3 43.4) (end 136.723 43.4) (width 0.2) (layer "F.Cu") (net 1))
 (segment (start 138.55 43.55) (end 147 52) (width 0.2) (layer "F.Cu") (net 1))
 (segment (start 126.72 43.4) (end 128.3 43.4) (width 0.2) (layer "F.Cu") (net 1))
 (segment (start 136.873 41.35) (end 138.677372 41.35) (width 0.2) (layer "F.Cu") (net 6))
 (segment (start 137.021 83.02) (end 137.021 83.8) (width 0.2) (layer "F.Cu") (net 6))
 (segment (start 113.048 56.508) (end 113.048 52.90424) (width 0.2) (layer "F.Cu") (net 6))
 (segment (start 128.3 41.7) (end 128.3 41.1) (width 0.2) (layer "F.Cu") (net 6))
 (segment (start 149.7 67.894) (end 150.7 68.894) (width 0.2) (layer "F.Cu") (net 6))
 (segment (start 114.36124 51.591) (end 117.909 51.591) (width 0.2) (layer "F.Cu") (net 6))
 (segment (start 114.6 58.06) (end 113.048 56.508) (width 0.2) (layer "F.Cu") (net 6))
 (segment (start 129.3 83.3) (end 136.821 83.3) (width 0.2) (layer "F.Cu") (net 6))
 (segment (start 128.1 41.1) (end 128.3 41.1) (width 0.2) (layer "F.Cu") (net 6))
 (segment (start 136.821 82.773) (end 136.821 83.3) (width 0.2) (layer "F.Cu") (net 6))
 (segment (start 117.909 51.591) (end 128.3 41.2) (width 0.2) (layer "F.Cu") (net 6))
 (segment (start 113.048 52.90424) (end 114.36124 51.591) (width 0.2) (layer "F.Cu") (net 6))
 (segment (start 138.677372 41.35) (end 149.7 52.372628) (width 0.2) (layer "F.Cu") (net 6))
 (segment (start 136.723 41.2) (end 136.873 41.35) (width 0.2) (layer "F.Cu") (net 6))
 (segment (start 150.7 68.894) (end 136.821 82.773) (width 0.2) (layer "F.Cu") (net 6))
 (segment (start 128.3 41.2) (end 136.723 41.2) (width 0.2) (layer "F.Cu") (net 6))
 (segment (start 149.7 52.372628) (end 149.7 67.894) (width 0.2) (layer "F.Cu") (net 6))
 (segment (start 145.62 69.921) (end 136.841 78.7) (width 0.2) (layer "F.Cu") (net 3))
 (segment (start 114.12324 56.671) (end 117.229 56.671) (width 0.2) (layer "F.Cu") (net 3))
 (segment (start 145.62 68.894) (end 145.62 69.921) (width 0.2) (layer "F.Cu") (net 3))
 (segment (start 128.4 45.5) (end 128.3 45.6) (width 0.2) (layer "F.Cu") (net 3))
 (segment (start 114.6 52.98) (end 113.449 54.131) (width 0.2) (layer "F.Cu") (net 3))
 (segment (start 128.3 45.6) (end 136.723 45.6) (width 0.2) (layer "F.Cu") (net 3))
 (segment (start 144.2 51.6) (end 144.2 67.474) (width 0.2) (layer "F.Cu") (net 3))
 (segment (start 113.449 54.131) (end 113.449 55.99676) (width 0.2) (layer "F.Cu") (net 3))
 (segment (start 138.35 45.75) (end 144.2 51.6) (width 0.2) (layer "F.Cu") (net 3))
 (segment (start 113.449 55.99676) (end 114.12324 56.671) (width 0.2) (layer "F.Cu") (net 3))
 (segment (start 117.229 56.671) (end 128.3 45.6) (width 0.2) (layer "F.Cu") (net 3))
 (segment (start 145.62 68.894) (end 145.6 68.914) (width 0.2) (layer "F.Cu") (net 3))
 (segment (start 129.32 78.8) (end 136.741 78.8) (width 0.2) (layer "F.Cu") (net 3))
 (segment (start 136.873 45.75) (end 138.35 45.75) (width 0.2) (layer "F.Cu") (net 3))
 (segment (start 136.941 79.2) (end 137.041 79.1) (width 0.2) (layer "F.Cu") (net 3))
 (segment (start 136.741 78.8) (end 136.841 78.7) (width 0.2) (layer "F.Cu") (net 3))
 (segment (start 136.821 79.1) (end 137.021 79.3) (width 0.2) (layer "F.Cu") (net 3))
 (segment (start 136.723 45.6) (end 136.873 45.75) (width 0.2) (layer "F.Cu") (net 3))
 (segment (start 144.2 67.474) (end 145.62 68.894) (width 0.2) (layer "F.Cu") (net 3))
 (segment (start 136.025 69.299) (end 135.62 68.894) (width 0.2) (layer "F.Cu") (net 16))
 (segment (start 136.025 72.75) (end 136.025 69.299) (width 0.2) (layer "F.Cu") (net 16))
 (segment (start 122.079 67.001) (end 122.14 66.94) (width 0.2) (layer "F.Cu") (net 8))
 (segment (start 138 53.4) (end 125.32 66.08) (width 0.2) (layer "F.Cu") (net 8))
 (segment (start 123 66.08) (end 122.079 67.001) (width 0.2) (layer "F.Cu") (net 8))
 (segment (start 118.461 67.001) (end 122.079 67.001) (width 0.2) (layer "F.Cu") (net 8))
 (segment (start 114.6 63.14) (end 118.461 67.001) (width 0.2) (layer "F.Cu") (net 8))
 (segment (start 125.32 66.08) (end 123 66.08) (width 0.2) (layer "F.Cu") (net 8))
 (segment (start 120.7 66) (end 133.3 53.4) (width 0.2) (layer "F.Cu") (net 7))
 (segment (start 133.3 53.4) (end 135.62 53.4) (width 0.2) (layer "F.Cu") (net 7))
 (segment (start 120 66) (end 120.7 66) (width 0.2) (layer "F.Cu") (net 7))
 (segment (start 114.6 60.6) (end 120 66) (width 0.2) (layer "F.Cu") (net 7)))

